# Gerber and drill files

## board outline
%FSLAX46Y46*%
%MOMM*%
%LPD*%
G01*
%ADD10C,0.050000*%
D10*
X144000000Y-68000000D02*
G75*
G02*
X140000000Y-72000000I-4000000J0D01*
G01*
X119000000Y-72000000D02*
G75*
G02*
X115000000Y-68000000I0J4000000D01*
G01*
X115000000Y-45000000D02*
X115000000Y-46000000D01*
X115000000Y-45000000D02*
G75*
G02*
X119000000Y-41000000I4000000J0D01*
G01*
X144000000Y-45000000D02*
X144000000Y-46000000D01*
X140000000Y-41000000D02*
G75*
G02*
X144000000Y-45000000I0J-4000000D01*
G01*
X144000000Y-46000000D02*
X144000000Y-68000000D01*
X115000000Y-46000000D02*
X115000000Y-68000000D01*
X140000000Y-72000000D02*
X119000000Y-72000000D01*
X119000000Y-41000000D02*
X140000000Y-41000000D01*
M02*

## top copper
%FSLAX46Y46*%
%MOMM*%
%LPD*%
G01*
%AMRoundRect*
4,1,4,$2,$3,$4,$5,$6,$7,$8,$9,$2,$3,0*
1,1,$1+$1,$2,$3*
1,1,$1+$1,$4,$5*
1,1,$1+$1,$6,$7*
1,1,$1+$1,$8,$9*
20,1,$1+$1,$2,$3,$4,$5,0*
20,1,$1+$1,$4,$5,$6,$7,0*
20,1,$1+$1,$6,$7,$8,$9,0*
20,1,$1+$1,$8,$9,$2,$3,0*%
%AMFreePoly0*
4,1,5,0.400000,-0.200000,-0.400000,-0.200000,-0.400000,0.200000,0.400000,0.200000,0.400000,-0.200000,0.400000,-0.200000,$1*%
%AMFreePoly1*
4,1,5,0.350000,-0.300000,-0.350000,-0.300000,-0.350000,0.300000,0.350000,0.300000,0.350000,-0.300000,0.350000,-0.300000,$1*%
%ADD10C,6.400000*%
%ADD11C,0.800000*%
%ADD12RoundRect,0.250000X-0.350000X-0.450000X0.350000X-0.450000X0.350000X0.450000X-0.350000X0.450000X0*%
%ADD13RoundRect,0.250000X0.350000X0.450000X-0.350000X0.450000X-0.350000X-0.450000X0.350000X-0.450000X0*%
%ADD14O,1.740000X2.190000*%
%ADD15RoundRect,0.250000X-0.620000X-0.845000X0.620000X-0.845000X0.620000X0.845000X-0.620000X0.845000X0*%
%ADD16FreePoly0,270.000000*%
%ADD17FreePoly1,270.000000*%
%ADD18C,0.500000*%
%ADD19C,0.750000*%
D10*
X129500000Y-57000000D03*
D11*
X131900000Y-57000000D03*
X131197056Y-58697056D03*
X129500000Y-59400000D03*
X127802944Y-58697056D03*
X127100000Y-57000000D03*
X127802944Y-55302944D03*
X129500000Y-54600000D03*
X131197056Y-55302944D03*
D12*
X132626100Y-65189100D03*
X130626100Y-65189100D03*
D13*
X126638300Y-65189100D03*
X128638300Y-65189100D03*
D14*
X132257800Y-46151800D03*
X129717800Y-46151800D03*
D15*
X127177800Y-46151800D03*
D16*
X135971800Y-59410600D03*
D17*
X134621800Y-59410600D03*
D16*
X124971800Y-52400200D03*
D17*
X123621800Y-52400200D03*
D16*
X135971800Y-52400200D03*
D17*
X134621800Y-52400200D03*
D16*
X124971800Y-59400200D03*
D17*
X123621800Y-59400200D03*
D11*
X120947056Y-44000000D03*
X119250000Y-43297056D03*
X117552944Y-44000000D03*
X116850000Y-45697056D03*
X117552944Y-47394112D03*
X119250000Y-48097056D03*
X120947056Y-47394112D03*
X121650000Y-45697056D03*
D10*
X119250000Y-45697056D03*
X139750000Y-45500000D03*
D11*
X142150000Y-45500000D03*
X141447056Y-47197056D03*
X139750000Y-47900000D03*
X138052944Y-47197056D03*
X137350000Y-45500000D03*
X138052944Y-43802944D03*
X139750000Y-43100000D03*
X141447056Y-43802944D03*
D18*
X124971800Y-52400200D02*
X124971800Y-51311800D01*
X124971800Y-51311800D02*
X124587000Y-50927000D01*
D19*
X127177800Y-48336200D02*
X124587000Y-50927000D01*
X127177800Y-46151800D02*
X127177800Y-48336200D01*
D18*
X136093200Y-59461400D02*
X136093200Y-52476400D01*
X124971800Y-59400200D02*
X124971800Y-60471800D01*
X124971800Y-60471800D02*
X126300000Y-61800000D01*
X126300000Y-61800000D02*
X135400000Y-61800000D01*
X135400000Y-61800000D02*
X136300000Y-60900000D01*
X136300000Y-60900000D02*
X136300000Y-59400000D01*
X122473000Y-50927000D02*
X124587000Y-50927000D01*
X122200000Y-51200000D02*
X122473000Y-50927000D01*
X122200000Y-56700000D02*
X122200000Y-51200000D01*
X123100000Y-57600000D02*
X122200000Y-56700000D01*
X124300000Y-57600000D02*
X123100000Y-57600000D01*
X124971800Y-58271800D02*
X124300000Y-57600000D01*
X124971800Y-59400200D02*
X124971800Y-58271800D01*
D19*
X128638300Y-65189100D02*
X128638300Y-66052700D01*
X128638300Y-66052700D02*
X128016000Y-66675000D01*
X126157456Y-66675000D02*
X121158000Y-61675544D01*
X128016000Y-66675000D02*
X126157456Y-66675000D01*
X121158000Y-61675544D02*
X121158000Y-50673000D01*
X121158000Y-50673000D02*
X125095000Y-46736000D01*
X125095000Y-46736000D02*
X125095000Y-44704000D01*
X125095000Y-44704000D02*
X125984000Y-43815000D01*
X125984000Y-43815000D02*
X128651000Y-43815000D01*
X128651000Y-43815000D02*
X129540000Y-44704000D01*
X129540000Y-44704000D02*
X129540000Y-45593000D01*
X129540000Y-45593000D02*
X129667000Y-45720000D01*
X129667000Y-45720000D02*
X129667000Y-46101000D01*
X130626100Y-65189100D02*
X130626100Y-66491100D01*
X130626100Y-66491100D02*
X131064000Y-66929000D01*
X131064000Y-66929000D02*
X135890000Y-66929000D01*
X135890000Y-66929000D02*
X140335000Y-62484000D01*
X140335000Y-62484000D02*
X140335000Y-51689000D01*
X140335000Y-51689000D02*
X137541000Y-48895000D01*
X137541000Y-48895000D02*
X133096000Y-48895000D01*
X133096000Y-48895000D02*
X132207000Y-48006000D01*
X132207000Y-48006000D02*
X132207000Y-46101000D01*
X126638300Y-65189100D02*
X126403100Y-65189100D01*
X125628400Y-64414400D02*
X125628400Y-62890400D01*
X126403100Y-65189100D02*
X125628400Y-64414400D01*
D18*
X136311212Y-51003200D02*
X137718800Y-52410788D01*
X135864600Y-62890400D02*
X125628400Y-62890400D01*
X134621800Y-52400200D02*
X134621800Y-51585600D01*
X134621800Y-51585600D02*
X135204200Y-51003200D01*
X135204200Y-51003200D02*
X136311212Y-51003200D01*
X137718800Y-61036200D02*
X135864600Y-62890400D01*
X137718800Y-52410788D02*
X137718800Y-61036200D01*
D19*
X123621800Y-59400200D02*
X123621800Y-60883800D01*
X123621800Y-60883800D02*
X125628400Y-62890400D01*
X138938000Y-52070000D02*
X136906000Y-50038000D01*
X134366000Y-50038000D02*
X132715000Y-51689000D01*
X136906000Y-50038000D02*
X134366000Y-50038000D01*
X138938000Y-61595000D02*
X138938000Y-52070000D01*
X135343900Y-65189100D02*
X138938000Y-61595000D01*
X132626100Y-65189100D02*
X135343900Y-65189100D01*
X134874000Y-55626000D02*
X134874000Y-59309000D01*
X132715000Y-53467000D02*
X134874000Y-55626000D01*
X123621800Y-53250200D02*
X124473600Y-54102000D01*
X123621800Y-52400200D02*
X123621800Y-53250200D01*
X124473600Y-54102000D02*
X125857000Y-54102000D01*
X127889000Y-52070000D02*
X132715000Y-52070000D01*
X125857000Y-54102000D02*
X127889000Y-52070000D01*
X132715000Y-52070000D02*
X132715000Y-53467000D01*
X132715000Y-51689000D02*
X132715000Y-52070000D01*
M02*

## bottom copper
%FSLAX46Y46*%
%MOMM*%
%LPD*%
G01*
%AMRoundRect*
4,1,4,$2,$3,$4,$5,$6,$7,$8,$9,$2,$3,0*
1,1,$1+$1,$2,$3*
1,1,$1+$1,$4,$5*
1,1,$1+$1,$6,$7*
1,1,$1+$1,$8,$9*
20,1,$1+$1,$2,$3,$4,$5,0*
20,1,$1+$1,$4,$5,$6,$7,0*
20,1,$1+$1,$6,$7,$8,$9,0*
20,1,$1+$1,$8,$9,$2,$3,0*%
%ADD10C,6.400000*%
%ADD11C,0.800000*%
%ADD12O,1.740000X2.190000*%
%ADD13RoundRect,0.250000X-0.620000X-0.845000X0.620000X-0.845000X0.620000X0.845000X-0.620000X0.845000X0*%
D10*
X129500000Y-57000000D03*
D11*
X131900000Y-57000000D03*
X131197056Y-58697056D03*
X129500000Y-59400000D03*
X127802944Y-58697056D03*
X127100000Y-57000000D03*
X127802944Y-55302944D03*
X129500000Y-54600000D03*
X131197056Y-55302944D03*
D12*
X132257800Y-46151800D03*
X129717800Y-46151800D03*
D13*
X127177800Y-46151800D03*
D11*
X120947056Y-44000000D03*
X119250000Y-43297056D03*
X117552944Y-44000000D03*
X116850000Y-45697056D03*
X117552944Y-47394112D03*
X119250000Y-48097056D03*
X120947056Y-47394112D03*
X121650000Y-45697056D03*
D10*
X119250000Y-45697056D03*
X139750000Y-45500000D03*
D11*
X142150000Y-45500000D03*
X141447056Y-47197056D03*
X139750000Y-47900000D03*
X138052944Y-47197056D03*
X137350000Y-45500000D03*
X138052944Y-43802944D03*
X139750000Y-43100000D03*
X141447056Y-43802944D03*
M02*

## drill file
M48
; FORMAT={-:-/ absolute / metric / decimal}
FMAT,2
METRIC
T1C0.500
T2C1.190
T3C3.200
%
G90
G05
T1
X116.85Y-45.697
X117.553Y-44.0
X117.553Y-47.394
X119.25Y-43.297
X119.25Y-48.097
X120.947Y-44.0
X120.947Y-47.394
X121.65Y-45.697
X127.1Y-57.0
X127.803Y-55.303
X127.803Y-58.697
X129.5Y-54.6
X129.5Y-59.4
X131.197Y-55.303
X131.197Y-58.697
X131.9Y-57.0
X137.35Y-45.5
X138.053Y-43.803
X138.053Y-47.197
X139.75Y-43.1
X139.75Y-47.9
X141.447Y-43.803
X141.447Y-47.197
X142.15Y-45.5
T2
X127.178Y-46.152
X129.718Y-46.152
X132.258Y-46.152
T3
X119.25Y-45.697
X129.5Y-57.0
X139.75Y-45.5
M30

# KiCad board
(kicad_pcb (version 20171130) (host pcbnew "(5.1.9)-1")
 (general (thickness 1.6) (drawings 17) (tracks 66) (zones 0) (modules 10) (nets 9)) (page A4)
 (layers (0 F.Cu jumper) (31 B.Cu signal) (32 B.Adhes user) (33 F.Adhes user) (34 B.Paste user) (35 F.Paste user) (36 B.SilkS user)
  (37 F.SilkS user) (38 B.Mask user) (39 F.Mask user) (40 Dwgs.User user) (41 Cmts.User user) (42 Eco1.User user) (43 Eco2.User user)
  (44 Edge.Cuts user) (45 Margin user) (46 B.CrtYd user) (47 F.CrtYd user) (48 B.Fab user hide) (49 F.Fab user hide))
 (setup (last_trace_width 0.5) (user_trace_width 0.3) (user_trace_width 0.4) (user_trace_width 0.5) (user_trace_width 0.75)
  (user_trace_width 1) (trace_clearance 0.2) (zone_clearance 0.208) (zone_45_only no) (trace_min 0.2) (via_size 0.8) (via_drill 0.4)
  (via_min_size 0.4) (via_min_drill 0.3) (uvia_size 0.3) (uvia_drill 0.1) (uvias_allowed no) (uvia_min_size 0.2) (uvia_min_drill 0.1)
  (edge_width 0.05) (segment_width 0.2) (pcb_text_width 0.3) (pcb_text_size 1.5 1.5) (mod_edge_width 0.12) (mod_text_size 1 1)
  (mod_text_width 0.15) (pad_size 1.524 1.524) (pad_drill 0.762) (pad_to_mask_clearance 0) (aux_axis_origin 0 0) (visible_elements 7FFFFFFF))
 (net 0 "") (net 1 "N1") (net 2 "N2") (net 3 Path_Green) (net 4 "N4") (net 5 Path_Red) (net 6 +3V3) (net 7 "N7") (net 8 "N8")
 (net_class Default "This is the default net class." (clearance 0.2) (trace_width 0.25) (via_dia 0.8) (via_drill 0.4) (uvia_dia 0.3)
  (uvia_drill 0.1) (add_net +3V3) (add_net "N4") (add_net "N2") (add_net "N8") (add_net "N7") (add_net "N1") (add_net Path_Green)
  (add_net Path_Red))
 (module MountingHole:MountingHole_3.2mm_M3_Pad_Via (layer F.Cu) (at 129.5 57)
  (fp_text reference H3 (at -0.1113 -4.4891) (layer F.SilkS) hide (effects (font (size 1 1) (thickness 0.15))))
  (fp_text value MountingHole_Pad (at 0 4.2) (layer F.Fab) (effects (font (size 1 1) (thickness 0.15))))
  (pad 1 thru_hole circle (at 0 0) (size 6.4 6.4) (drill 3.2) (layers *.Cu *.Mask) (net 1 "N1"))
  (pad 1 thru_hole circle (at 2.4 0) (size 0.8 0.8) (drill 0.5) (layers *.Cu *.Mask) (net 1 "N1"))
  (pad 1 thru_hole circle (at 1.697056 1.697056) (size 0.8 0.8) (drill 0.5) (layers *.Cu *.Mask) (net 1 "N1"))
  (pad 1 thru_hole circle (at 0 2.4) (size 0.8 0.8) (drill 0.5) (layers *.Cu *.Mask) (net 1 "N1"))
  (pad 1 thru_hole circle (at -1.697056 1.697056) (size 0.8 0.8) (drill 0.5) (layers *.Cu *.Mask) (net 1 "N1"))
  (pad 1 thru_hole circle (at -2.4 0) (size 0.8 0.8) (drill 0.5) (layers *.Cu *.Mask) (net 1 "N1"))
  (pad 1 thru_hole circle (at -1.697056 -1.697056) (size 0.8 0.8) (drill 0.5) (layers *.Cu *.Mask) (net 1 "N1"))
  (pad 1 thru_hole circle (at 0 -2.4) (size 0.8 0.8) (drill 0.5) (layers *.Cu *.Mask) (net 1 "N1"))
  (pad 1 thru_hole circle (at 1.697056 -1.697056) (size 0.8 0.8) (drill 0.5) (layers *.Cu *.Mask) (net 1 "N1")))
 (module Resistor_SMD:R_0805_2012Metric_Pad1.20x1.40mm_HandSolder (layer F.Cu) (at 131.6261 65.1891)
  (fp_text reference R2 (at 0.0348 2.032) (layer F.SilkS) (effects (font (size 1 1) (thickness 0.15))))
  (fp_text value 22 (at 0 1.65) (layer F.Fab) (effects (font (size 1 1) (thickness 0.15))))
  (pad 2 smd roundrect (at 1 0) (size 1.2 1.4) (layers F.Cu F.Paste F.Mask) (roundrect_rratio 0.208333) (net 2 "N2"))
  (pad 1 smd roundrect (at -1 0) (size 1.2 1.4) (layers F.Cu F.Paste F.Mask) (roundrect_rratio 0.208333) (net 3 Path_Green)))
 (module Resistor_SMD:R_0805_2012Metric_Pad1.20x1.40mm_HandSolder (layer F.Cu) (at 127.6383 65.1891 180)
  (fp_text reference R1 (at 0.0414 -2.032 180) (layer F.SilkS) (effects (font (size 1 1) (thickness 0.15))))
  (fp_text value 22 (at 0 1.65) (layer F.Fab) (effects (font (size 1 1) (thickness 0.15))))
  (pad 2 smd roundrect (at 1 0 180) (size 1.2 1.4) (layers F.Cu F.Paste F.Mask) (roundrect_rratio 0.208333) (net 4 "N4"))
  (pad 1 smd roundrect (at -1 0 180) (size 1.2 1.4) (layers F.Cu F.Paste F.Mask) (roundrect_rratio 0.208333) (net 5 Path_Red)))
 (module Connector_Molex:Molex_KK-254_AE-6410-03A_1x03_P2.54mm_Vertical (layer F.Cu) (at 127.1778 46.1518)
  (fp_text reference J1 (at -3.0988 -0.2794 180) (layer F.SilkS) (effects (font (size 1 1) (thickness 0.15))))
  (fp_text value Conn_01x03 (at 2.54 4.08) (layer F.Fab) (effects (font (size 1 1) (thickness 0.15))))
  (pad 3 thru_hole oval (at 5.08 0) (size 1.74 2.19) (drill 1.19) (layers *.Cu *.Mask) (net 3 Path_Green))
  (pad 2 thru_hole oval (at 2.54 0) (size 1.74 2.19) (drill 1.19) (layers *.Cu *.Mask) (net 5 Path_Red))
  (pad 1 thru_hole roundrect (at 0 0) (size 1.74 2.19) (drill 1.19) (layers *.Cu *.Mask) (roundrect_rratio 0.143678) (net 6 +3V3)))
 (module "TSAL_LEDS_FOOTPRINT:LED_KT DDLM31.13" (layer F.Cu) (at 135.2468 59.3856 270)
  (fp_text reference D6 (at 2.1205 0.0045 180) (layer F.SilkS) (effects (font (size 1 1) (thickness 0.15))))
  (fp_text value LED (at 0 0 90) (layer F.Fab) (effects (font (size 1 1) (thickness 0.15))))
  (pad 2 smd custom (at 0.025 -0.725 270) (size 0.8 0.4) (layers F.Cu F.Paste F.Mask) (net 6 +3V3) (zone_connect 0)
   (options (clearance outline) (anchor rect)) (primitives))
  (pad 1 smd custom (at 0.025 0.625 270) (size 0.7 0.6) (layers F.Cu F.Paste F.Mask) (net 2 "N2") (zone_connect 0)
   (options (clearance outline) (anchor rect)) (primitives)))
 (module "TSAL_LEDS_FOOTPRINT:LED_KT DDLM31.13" (layer F.Cu) (at 124.2468 52.3752 270)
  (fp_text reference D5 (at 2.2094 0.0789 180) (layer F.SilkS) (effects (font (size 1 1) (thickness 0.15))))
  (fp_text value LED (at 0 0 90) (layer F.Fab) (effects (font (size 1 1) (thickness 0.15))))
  (pad 2 smd custom (at 0.025 -0.725 270) (size 0.8 0.4) (layers F.Cu F.Paste F.Mask) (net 6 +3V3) (zone_connect 0)
   (options (clearance outline) (anchor rect)) (primitives))
  (pad 1 smd custom (at 0.025 0.625 270) (size 0.7 0.6) (layers F.Cu F.Paste F.Mask) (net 2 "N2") (zone_connect 0)
   (options (clearance outline) (anchor rect)) (primitives)))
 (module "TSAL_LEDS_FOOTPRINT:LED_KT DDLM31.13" (layer F.Cu) (at 135.2468 52.3752 270)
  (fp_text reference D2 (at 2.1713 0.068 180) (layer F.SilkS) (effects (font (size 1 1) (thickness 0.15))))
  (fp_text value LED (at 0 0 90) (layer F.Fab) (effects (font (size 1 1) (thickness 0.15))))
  (pad 2 smd custom (at 0.025 -0.725 270) (size 0.8 0.4) (layers F.Cu F.Paste F.Mask) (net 6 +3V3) (zone_connect 0)
   (options (clearance outline) (anchor rect)) (primitives))
  (pad 1 smd custom (at 0.025 0.625 270) (size 0.7 0.6) (layers F.Cu F.Paste F.Mask) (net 4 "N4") (zone_connect 0)
   (options (clearance outline) (anchor rect)) (primitives)))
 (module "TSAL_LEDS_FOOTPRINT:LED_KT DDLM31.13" (layer F.Cu) (at 124.2468 59.3752 270)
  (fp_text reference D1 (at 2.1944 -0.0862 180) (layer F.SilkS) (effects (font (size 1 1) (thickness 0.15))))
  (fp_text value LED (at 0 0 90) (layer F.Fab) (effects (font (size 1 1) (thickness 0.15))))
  (pad 2 smd custom (at 0.025 -0.725 270) (size 0.8 0.4) (layers F.Cu F.Paste F.Mask) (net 6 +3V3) (zone_connect 0)
   (options (clearance outline) (anchor rect)) (primitives))
  (pad 1 smd custom (at 0.025 0.625 270) (size 0.7 0.6) (layers F.Cu F.Paste F.Mask) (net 4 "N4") (zone_connect 0)
   (options (clearance outline) (anchor rect)) (primitives)))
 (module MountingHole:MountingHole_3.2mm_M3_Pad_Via (layer F.Cu) (at 119.25 45.697056)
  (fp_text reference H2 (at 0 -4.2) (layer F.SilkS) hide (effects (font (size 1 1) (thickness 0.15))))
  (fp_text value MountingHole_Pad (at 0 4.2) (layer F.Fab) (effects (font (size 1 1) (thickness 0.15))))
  (pad 1 thru_hole circle (at 1.697056 -1.697056) (size 0.8 0.8) (drill 0.5) (layers *.Cu *.Mask) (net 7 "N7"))
  (pad 1 thru_hole circle (at 0 -2.4) (size 0.8 0.8) (drill 0.5) (layers *.Cu *.Mask) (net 7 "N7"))
  (pad 1 thru_hole circle (at -1.697056 -1.697056) (size 0.8 0.8) (drill 0.5) (layers *.Cu *.Mask) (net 7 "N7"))
  (pad 1 thru_hole circle (at -2.4 0) (size 0.8 0.8) (drill 0.5) (layers *.Cu *.Mask) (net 7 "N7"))
  (pad 1 thru_hole circle (at -1.697056 1.697056) (size 0.8 0.8) (drill 0.5) (layers *.Cu *.Mask) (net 7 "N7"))
  (pad 1 thru_hole circle (at 0 2.4) (size 0.8 0.8) (drill 0.5) (layers *.Cu *.Mask) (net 7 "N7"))
  (pad 1 thru_hole circle (at 1.697056 1.697056) (size 0.8 0.8) (drill 0.5) (layers *.Cu *.Mask) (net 7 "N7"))
  (pad 1 thru_hole circle (at 2.4 0) (size 0.8 0.8) (drill 0.5) (layers *.Cu *.Mask) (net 7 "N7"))
  (pad 1 thru_hole circle (at 0 0) (size 6.4 6.4) (drill 3.2) (layers *.Cu *.Mask) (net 7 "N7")))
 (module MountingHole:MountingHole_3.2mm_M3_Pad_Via (layer F.Cu) (at 139.75 45.5)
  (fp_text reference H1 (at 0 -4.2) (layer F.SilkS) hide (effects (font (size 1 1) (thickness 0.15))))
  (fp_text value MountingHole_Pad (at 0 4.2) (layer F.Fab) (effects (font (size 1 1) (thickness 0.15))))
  (pad 1 thru_hole circle (at 0 0) (size 6.4 6.4) (drill 3.2) (layers *.Cu *.Mask) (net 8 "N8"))
  (pad 1 thru_hole circle (at 2.4 0) (size 0.8 0.8) (drill 0.5) (layers *.Cu *.Mask) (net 8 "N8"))
  (pad 1 thru_hole circle (at 1.697056 1.697056) (size 0.8 0.8) (drill 0.5) (layers *.Cu *.Mask) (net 8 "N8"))
  (pad 1 thru_hole circle (at 0 2.4) (size 0.8 0.8) (drill 0.5) (layers *.Cu *.Mask) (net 8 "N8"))
  (pad 1 thru_hole circle (at -1.697056 1.697056) (size 0.8 0.8) (drill 0.5) (layers *.Cu *.Mask) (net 8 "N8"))
  (pad 1 thru_hole circle (at -2.4 0) (size 0.8 0.8) (drill 0.5) (layers *.Cu *.Mask) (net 8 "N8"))
  (pad 1 thru_hole circle (at -1.697056 -1.697056) (size 0.8 0.8) (drill 0.5) (layers *.Cu *.Mask) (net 8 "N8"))
  (pad 1 thru_hole circle (at 0 -2.4) (size 0.8 0.8) (drill 0.5) (layers *.Cu *.Mask) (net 8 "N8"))
  (pad 1 thru_hole circle (at 1.697056 -1.697056) (size 0.8 0.8) (drill 0.5) (layers *.Cu *.Mask) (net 8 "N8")))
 (gr_arc (start 140 68) (end 140 72) (angle -90) (layer Edge.Cuts) (width 0.05))
 (gr_arc (start 119 68) (end 115 68) (angle -90) (layer Edge.Cuts) (width 0.05))
 (gr_line (start 115 45) (end 115 46) (layer Edge.Cuts) (width 0.05))
 (gr_arc (start 119 45) (end 119 41) (angle -90) (layer Edge.Cuts) (width 0.05))
 (gr_line (start 144 45) (end 144 46) (layer Edge.Cuts) (width 0.05))
 (gr_arc (start 140 45) (end 144 45) (angle -90) (layer Edge.Cuts) (width 0.05))
 (gr_line (start 144 46) (end 144 68) (layer Edge.Cuts) (width 0.05))
 (gr_line (start 115 46) (end 115 68) (layer Edge.Cuts) (width 0.05))
 (gr_line (start 140 72) (end 119 72) (layer Edge.Cuts) (width 0.05))
 (gr_line (start 119 41) (end 140 41) (layer Edge.Cuts) (width 0.05))
 (segment (start 124.9718 52.4002) (end 124.9718 51.3118) (width 0.5) (layer F.Cu) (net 6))
 (segment (start 124.9718 51.3118) (end 124.587 50.927) (width 0.5) (layer F.Cu) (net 6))
 (segment (start 127.1778 48.3362) (end 124.587 50.927) (width 0.75) (layer F.Cu) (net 6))
 (segment (start 127.1778 46.1518) (end 127.1778 48.3362) (width 0.75) (layer F.Cu) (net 6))
 (segment (start 136.0932 59.4614) (end 136.0932 52.4764) (width 0.5) (layer F.Cu) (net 6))
 (segment (start 124.9718 59.4002) (end 124.9718 60.4718) (width 0.5) (layer F.Cu) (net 6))
 (segment (start 124.9718 60.4718) (end 126.3 61.8) (width 0.5) (layer F.Cu) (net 6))
 (segment (start 126.3 61.8) (end 135.4 61.8) (width 0.5) (layer F.Cu) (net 6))
 (segment (start 135.4 61.8) (end 136.3 60.9) (width 0.5) (layer F.Cu) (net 6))
 (segment (start 136.3 60.9) (end 136.3 59.4) (width 0.5) (layer F.Cu) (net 6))
 (segment (start 122.473 50.927) (end 124.587 50.927) (width 0.5) (layer F.Cu) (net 6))
 (segment (start 122.2 51.2) (end 122.473 50.927) (width 0.5) (layer F.Cu) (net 6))
 (segment (start 122.2 56.7) (end 122.2 51.2) (width 0.5) (layer F.Cu) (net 6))
 (segment (start 123.1 57.6) (end 122.2 56.7) (width 0.5) (layer F.Cu) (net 6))
 (segment (start 124.3 57.6) (end 123.1 57.6) (width 0.5) (layer F.Cu) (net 6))
 (segment (start 124.9718 58.2718) (end 124.3 57.6) (width 0.5) (layer F.Cu) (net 6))
 (segment (start 124.9718 59.4002) (end 124.9718 58.2718) (width 0.5) (layer F.Cu) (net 6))
 (segment (start 128.6383 65.1891) (end 128.6383 66.0527) (width 0.75) (layer F.Cu) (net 5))
 (segment (start 128.6383 66.0527) (end 128.016 66.675) (width 0.75) (layer F.Cu) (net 5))
 (segment (start 126.157456 66.675) (end 121.158 61.675544) (width 0.75) (layer F.Cu) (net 5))
 (segment (start 128.016 66.675) (end 126.157456 66.675) (width 0.75) (layer F.Cu) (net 5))
 (segment (start 121.158 61.675544) (end 121.158 50.673) (width 0.75) (layer F.Cu) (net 5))
 (segment (start 121.158 50.673) (end 125.095 46.736) (width 0.75) (layer F.Cu) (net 5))
 (segment (start 125.095 46.736) (end 125.095 44.704) (width 0.75) (layer F.Cu) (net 5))
 (segment (start 125.095 44.704) (end 125.984 43.815) (width 0.75) (layer F.Cu) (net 5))
 (segment (start 125.984 43.815) (end 128.651 43.815) (width 0.75) (layer F.Cu) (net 5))
 (segment (start 128.651 43.815) (end 129.54 44.704) (width 0.75) (layer F.Cu) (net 5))
 (segment (start 129.54 44.704) (end 129.54 45.593) (width 0.75) (layer F.Cu) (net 5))
 (segment (start 129.54 45.593) (end 129.667 45.72) (width 0.75) (layer F.Cu) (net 5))
 (segment (start 129.667 45.72) (end 129.667 46.101) (width 0.75) (layer F.Cu) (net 5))
 (segment (start 130.6261 65.1891) (end 130.6261 66.4911) (width 0.75) (layer F.Cu) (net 3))
 (segment (start 130.6261 66.4911) (end 131.064 66.929) (width 0.75) (layer F.Cu) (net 3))
 (segment (start 131.064 66.929) (end 135.89 66.929) (width 0.75) (layer F.Cu) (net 3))
 (segment (start 135.89 66.929) (end 140.335 62.484) (width 0.75) (layer F.Cu) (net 3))
 (segment (start 140.335 62.484) (end 140.335 51.689) (width 0.75) (layer F.Cu) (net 3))
 (segment (start 140.335 51.689) (end 137.541 48.895) (width 0.75) (layer F.Cu) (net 3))
 (segment (start 137.541 48.895) (end 133.096 48.895) (width 0.75) (layer F.Cu) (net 3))
 (segment (start 133.096 48.895) (end 132.207 48.006) (width 0.75) (layer F.Cu) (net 3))
 (segment (start 132.207 48.006) (end 132.207 46.101) (width 0.75) (layer F.Cu) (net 3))
 (segment (start 126.6383 65.1891) (end 126.4031 65.1891) (width 0.75) (layer F.Cu) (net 4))
 (segment (start 125.6284 64.4144) (end 125.6284 62.8904) (width 0.75) (layer F.Cu) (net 4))
 (segment (start 126.4031 65.1891) (end 125.6284 64.4144) (width 0.75) (layer F.Cu) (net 4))
 (segment (start 136.311212 51.0032) (end 137.7188 52.410788) (width 0.5) (layer F.Cu) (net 4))
 (segment (start 135.8646 62.8904) (end 125.6284 62.8904) (width 0.5) (layer F.Cu) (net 4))
 (segment (start 134.6218 52.4002) (end 134.6218 51.5856) (width 0.5) (layer F.Cu) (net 4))
 (segment (start 134.6218 51.5856) (end 135.2042 51.0032) (width 0.5) (layer F.Cu) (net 4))
 (segment (start 135.2042 51.0032) (end 136.311212 51.0032) (width 0.5) (layer F.Cu) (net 4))
 (segment (start 137.7188 61.0362) (end 135.8646 62.8904) (width 0.5) (layer F.Cu) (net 4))
 (segment (start 137.7188 52.410788) (end 137.7188 61.0362) (width 0.5) (layer F.Cu) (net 4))
 (segment (start 123.6218 59.4002) (end 123.6218 60.8838) (width 0.75) (layer F.Cu) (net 4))
 (segment (start 123.6218 60.8838) (end 125.6284 62.8904) (width 0.75) (layer F.Cu) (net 4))
 (segment (start 138.938 52.07) (end 136.906 50.038) (width 0.75) (layer F.Cu) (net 2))
 (segment (start 134.366 50.038) (end 132.715 51.689) (width 0.75) (layer F.Cu) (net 2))
 (segment (start 136.906 50.038) (end 134.366 50.038) (width 0.75) (layer F.Cu) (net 2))
 (segment (start 138.938 61.595) (end 138.938 52.07) (width 0.75) (layer F.Cu) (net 2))
 (segment (start 135.3439 65.1891) (end 138.938 61.595) (width 0.75) (layer F.Cu) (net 2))
 (segment (start 132.6261 65.1891) (end 135.3439 65.1891) (width 0.75) (layer F.Cu) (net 2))
 (segment (start 134.874 55.626) (end 134.874 59.309) (width 0.75) (layer F.Cu) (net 2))
 (segment (start 132.715 53.467) (end 134.874 55.626) (width 0.75) (layer F.Cu) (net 2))
 (segment (start 123.6218 53.2502) (end 124.4736 54.102) (width 0.75) (layer F.Cu) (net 2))
 (segment (start 123.6218 52.4002) (end 123.6218 53.2502) (width 0.75) (layer F.Cu) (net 2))
 (segment (start 124.4736 54.102) (end 125.857 54.102) (width 0.75) (layer F.Cu) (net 2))
 (segment (start 127.889 52.07) (end 132.715 52.07) (width 0.75) (layer F.Cu) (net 2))
 (segment (start 125.857 54.102) (end 127.889 52.07) (width 0.75) (layer F.Cu) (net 2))
 (segment (start 132.715 52.07) (end 132.715 53.467) (width 0.75) (layer F.Cu) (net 2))
 (segment (start 132.715 51.689) (end 132.715 52.07) (width 0.75) (layer F.Cu) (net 2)))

